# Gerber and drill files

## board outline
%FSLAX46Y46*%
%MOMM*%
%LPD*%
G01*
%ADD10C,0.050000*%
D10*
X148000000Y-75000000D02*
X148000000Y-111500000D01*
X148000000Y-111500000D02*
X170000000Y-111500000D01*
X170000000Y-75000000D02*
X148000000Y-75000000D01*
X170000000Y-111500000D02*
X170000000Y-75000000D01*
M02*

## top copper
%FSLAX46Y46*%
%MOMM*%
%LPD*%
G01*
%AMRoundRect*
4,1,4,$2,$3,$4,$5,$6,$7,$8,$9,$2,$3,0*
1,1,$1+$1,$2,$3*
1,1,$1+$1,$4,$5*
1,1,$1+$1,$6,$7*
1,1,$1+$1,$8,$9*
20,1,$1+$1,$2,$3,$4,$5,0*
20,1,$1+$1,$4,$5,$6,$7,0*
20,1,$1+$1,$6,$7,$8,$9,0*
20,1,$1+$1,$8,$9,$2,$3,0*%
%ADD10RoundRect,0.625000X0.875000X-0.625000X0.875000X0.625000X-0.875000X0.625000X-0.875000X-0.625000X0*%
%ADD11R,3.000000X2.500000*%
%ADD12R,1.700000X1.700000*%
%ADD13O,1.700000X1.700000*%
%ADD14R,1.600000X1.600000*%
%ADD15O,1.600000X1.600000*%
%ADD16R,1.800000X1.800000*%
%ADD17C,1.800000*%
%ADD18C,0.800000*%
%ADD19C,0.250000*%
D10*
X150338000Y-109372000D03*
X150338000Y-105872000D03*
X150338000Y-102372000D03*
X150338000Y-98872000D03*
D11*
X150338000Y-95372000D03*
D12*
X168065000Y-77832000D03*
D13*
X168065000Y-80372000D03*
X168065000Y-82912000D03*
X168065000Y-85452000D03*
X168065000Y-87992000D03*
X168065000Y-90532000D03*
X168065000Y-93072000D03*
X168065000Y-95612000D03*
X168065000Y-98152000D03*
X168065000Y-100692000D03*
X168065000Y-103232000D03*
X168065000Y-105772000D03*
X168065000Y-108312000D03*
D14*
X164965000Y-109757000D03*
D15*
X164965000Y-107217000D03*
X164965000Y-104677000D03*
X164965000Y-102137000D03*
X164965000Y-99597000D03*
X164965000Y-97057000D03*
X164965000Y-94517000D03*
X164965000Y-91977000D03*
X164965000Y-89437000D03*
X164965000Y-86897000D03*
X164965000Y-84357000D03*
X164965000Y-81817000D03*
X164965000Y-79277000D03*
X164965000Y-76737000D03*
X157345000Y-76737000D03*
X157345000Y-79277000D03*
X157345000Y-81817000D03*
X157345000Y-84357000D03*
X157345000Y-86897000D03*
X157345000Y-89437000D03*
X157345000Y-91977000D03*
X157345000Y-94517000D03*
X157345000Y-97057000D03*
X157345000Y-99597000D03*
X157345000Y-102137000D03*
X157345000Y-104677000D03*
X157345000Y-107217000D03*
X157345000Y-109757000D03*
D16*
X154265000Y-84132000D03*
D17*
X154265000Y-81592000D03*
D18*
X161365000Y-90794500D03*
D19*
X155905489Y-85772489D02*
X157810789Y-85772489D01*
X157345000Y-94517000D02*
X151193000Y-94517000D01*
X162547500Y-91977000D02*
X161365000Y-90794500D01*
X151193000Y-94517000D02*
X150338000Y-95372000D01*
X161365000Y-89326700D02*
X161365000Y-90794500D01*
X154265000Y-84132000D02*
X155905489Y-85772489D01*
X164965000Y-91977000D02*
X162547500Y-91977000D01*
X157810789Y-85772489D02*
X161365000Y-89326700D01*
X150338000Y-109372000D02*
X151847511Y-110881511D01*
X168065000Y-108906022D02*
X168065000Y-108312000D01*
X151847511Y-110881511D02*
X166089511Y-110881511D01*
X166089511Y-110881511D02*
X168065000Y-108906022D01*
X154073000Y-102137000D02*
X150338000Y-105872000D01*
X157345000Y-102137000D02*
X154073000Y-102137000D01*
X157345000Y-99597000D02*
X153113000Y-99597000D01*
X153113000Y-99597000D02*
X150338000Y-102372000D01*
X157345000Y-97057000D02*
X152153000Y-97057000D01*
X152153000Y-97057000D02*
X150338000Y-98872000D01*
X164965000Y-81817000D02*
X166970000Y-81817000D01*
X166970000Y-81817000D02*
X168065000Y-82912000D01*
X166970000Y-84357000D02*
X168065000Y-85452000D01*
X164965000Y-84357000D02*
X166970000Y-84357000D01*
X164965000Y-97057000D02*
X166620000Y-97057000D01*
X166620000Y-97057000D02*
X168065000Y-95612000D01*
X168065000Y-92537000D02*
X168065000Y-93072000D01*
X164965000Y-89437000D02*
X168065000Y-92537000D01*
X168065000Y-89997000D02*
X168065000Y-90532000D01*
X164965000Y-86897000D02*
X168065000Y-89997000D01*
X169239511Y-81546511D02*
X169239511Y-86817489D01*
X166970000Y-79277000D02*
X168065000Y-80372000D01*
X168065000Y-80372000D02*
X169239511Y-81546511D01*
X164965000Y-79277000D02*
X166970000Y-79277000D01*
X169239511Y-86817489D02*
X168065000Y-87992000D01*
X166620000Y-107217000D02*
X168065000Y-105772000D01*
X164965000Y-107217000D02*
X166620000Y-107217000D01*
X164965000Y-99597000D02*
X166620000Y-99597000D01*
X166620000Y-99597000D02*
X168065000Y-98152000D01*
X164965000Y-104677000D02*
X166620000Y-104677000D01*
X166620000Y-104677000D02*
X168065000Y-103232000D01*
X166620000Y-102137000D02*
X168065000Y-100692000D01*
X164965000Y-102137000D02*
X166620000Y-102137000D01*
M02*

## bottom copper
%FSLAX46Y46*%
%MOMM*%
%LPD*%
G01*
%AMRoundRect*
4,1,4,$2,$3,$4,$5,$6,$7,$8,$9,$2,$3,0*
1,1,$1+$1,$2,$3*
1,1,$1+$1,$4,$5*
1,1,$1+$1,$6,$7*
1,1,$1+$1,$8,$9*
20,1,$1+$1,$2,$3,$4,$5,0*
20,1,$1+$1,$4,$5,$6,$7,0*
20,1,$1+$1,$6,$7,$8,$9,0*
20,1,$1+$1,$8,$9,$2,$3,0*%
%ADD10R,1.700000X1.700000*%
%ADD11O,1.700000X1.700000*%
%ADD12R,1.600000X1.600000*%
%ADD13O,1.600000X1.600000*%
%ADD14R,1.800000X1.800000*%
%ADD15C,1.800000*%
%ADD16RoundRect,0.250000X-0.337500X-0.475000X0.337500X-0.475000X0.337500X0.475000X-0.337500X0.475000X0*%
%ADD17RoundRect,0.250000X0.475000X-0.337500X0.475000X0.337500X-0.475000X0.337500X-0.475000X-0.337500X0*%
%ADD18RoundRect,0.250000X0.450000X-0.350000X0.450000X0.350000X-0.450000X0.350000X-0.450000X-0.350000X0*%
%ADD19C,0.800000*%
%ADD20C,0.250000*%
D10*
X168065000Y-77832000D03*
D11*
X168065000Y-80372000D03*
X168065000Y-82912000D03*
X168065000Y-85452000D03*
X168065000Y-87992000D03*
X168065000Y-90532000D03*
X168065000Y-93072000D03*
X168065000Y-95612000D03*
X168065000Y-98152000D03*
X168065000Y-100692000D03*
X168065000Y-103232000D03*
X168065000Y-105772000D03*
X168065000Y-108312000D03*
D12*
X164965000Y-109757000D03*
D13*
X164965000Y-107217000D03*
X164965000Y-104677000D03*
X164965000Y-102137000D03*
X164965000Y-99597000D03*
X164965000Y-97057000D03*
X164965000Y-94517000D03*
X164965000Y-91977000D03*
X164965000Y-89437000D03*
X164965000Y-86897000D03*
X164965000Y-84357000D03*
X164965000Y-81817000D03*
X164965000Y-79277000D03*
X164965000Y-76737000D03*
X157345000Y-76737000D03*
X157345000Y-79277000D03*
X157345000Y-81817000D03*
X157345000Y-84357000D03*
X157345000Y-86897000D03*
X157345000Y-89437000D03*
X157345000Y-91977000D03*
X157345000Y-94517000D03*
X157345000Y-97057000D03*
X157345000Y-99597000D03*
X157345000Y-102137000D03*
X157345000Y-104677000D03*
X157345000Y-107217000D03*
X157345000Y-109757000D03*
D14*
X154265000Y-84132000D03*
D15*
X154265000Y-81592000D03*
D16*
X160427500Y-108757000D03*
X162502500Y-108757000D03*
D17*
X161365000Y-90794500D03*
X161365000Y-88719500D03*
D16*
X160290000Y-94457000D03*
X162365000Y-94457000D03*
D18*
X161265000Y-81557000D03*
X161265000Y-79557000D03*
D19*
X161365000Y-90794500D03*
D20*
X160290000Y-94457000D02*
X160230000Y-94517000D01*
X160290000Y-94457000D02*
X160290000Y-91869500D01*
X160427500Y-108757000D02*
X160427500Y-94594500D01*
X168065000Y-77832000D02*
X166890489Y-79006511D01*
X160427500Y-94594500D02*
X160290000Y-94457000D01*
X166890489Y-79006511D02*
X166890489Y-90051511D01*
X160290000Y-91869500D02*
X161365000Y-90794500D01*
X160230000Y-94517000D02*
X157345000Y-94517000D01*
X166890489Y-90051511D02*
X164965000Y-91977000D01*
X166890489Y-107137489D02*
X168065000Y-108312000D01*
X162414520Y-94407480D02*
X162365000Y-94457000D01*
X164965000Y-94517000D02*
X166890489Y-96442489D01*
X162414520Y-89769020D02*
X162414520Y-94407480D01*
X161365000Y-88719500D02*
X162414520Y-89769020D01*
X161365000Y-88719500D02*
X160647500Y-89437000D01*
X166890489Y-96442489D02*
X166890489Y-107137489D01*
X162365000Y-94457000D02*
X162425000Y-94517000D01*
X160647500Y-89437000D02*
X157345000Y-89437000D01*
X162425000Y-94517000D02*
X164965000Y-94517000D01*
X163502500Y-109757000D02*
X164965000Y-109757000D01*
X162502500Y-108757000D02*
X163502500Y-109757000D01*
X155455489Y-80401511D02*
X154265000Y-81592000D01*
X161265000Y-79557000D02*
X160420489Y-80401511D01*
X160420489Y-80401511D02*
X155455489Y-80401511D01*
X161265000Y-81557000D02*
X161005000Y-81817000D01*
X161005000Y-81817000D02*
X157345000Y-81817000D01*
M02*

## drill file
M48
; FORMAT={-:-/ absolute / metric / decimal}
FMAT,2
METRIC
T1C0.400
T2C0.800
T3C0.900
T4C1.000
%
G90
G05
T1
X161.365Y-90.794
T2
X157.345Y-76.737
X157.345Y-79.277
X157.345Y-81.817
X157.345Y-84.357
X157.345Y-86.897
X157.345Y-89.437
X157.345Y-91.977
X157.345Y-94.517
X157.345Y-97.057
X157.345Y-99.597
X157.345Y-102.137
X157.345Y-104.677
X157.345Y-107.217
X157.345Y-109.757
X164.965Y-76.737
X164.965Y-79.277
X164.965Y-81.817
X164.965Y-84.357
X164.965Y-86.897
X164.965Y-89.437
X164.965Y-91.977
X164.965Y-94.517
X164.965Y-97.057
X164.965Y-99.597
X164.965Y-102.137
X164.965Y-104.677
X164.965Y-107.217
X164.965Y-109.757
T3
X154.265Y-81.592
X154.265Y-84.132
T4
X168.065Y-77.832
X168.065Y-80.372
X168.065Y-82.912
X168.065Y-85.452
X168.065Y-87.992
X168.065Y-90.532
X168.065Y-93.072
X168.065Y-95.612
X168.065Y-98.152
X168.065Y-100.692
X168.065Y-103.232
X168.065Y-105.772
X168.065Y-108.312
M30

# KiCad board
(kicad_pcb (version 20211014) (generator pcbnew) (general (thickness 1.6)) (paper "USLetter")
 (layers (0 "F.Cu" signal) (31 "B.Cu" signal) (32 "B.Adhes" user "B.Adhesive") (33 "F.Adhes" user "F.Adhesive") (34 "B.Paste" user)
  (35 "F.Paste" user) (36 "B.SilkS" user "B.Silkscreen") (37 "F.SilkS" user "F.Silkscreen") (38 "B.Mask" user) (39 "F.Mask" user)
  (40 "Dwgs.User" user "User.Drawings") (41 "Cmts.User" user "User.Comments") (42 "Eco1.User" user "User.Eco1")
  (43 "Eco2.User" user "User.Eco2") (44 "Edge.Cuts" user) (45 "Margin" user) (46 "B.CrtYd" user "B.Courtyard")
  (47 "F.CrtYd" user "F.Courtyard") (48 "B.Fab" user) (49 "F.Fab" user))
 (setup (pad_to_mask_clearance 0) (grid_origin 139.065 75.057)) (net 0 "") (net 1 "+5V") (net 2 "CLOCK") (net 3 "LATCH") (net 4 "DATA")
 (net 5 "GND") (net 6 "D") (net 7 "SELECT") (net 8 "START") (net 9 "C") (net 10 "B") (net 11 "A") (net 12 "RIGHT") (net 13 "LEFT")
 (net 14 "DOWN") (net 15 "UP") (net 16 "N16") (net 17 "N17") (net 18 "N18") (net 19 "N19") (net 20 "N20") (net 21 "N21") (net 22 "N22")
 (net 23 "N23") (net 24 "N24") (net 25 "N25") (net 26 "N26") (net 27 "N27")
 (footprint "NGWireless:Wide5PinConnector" (layer "F.Cu") (at 150.465 102.357 90)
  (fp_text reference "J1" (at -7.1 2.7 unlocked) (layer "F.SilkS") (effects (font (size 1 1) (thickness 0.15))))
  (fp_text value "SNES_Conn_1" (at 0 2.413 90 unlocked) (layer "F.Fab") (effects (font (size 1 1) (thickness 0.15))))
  (pad "1" smd roundrect (at -7.015 -0.127 90) (size 2.5 3) (layers "F.Cu" "F.Paste" "F.Mask") (roundrect_rratio 0.25) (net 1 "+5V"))
  (pad "2" smd roundrect (at -3.515 -0.127 90) (size 2.5 3) (layers "F.Cu" "F.Paste" "F.Mask") (roundrect_rratio 0.25) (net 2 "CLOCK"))
  (pad "3" smd roundrect (at -0.015 -0.127 90) (size 2.5 3) (layers "F.Cu" "F.Paste" "F.Mask") (roundrect_rratio 0.25) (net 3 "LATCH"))
  (pad "4" smd roundrect (at 3.485 -0.127 90) (size 2.5 3) (layers "F.Cu" "F.Paste" "F.Mask") (roundrect_rratio 0.25) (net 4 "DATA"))
  (pad "5" smd rect (at 6.985 -0.127 90) (size 2.5 3) (layers "F.Cu" "F.Paste" "F.Mask") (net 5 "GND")))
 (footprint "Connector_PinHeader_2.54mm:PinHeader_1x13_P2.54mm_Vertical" (layer "F.Cu") (at 168.065 77.832)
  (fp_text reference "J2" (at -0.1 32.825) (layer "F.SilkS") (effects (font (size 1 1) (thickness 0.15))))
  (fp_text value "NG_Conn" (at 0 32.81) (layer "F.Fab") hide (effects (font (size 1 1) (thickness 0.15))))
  (pad "1" thru_hole rect locked (at 0 0) (size 1.7 1.7) (drill 1) (layers *.Cu *.Mask) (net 5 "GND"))
  (pad "2" thru_hole oval locked (at 0 2.54) (size 1.7 1.7) (drill 1) (layers *.Cu *.Mask) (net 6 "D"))
  (pad "3" thru_hole oval locked (at 0 5.08) (size 1.7 1.7) (drill 1) (layers *.Cu *.Mask) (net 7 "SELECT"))
  (pad "4" thru_hole oval locked (at 0 7.62) (size 1.7 1.7) (drill 1) (layers *.Cu *.Mask) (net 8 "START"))
  (pad "5" thru_hole oval locked (at 0 10.16) (size 1.7 1.7) (drill 1) (layers *.Cu *.Mask) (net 6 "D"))
  (pad "6" thru_hole oval locked (at 0 12.7) (size 1.7 1.7) (drill 1) (layers *.Cu *.Mask) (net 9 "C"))
  (pad "7" thru_hole oval locked (at 0 15.24) (size 1.7 1.7) (drill 1) (layers *.Cu *.Mask) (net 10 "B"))
  (pad "8" thru_hole oval locked (at 0 17.78) (size 1.7 1.7) (drill 1) (layers *.Cu *.Mask) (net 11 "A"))
  (pad "9" thru_hole oval locked (at 0 20.32) (size 1.7 1.7) (drill 1) (layers *.Cu *.Mask) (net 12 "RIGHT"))
  (pad "10" thru_hole oval locked (at 0 22.86) (size 1.7 1.7) (drill 1) (layers *.Cu *.Mask) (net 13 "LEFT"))
  (pad "11" thru_hole oval locked (at 0 25.4) (size 1.7 1.7) (drill 1) (layers *.Cu *.Mask) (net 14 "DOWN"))
  (pad "12" thru_hole oval locked (at 0 27.94) (size 1.7 1.7) (drill 1) (layers *.Cu *.Mask) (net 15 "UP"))
  (pad "13" thru_hole oval locked (at 0 30.48) (size 1.7 1.7) (drill 1) (layers *.Cu *.Mask) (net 1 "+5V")))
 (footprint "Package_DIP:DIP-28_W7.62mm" (layer "F.Cu") (at 164.965 109.757 180)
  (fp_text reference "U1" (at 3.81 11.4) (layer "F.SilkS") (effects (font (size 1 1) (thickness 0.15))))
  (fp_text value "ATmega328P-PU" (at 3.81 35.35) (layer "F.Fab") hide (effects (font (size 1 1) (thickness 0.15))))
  (pad "1" thru_hole rect locked (at 0 0 180) (size 1.6 1.6) (drill 0.8) (layers *.Cu *.Mask) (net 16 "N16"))
  (pad "2" thru_hole oval locked (at 0 2.54 180) (size 1.6 1.6) (drill 0.8) (layers *.Cu *.Mask) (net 15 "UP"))
  (pad "3" thru_hole oval locked (at 0 5.08 180) (size 1.6 1.6) (drill 0.8) (layers *.Cu *.Mask) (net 14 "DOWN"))
  (pad "4" thru_hole oval locked (at 0 7.62 180) (size 1.6 1.6) (drill 0.8) (layers *.Cu *.Mask) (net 13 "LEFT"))
  (pad "5" thru_hole oval locked (at 0 10.16 180) (size 1.6 1.6) (drill 0.8) (layers *.Cu *.Mask) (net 12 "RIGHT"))
  (pad "6" thru_hole oval locked (at 0 12.7 180) (size 1.6 1.6) (drill 0.8) (layers *.Cu *.Mask) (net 11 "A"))
  (pad "7" thru_hole oval locked (at 0 15.24 180) (size 1.6 1.6) (drill 0.8) (layers *.Cu *.Mask) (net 1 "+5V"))
  (pad "8" thru_hole oval locked (at 0 17.78 180) (size 1.6 1.6) (drill 0.8) (layers *.Cu *.Mask) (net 5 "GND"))
  (pad "9" thru_hole oval locked (at 0 20.32 180) (size 1.6 1.6) (drill 0.8) (layers *.Cu *.Mask) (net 10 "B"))
  (pad "10" thru_hole oval locked (at 0 22.86 180) (size 1.6 1.6) (drill 0.8) (layers *.Cu *.Mask) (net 9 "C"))
  (pad "11" thru_hole oval locked (at 0 25.4 180) (size 1.6 1.6) (drill 0.8) (layers *.Cu *.Mask) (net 8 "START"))
  (pad "12" thru_hole oval locked (at 0 27.94 180) (size 1.6 1.6) (drill 0.8) (layers *.Cu *.Mask) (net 7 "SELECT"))
  (pad "13" thru_hole oval locked (at 0 30.48 180) (size 1.6 1.6) (drill 0.8) (layers *.Cu *.Mask) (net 6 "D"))
  (pad "14" thru_hole oval locked (at 0 33.02 180) (size 1.6 1.6) (drill 0.8) (layers *.Cu *.Mask) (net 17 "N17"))
  (pad "15" thru_hole oval locked (at 7.62 33.02 180) (size 1.6 1.6) (drill 0.8) (layers *.Cu *.Mask) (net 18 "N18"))
  (pad "16" thru_hole oval locked (at 7.62 30.48 180) (size 1.6 1.6) (drill 0.8) (layers *.Cu *.Mask) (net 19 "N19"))
  (pad "17" thru_hole oval locked (at 7.62 27.94 180) (size 1.6 1.6) (drill 0.8) (layers *.Cu *.Mask) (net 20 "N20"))
  (pad "18" thru_hole oval locked (at 7.62 25.4 180) (size 1.6 1.6) (drill 0.8) (layers *.Cu *.Mask) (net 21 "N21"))
  (pad "19" thru_hole oval locked (at 7.62 22.86 180) (size 1.6 1.6) (drill 0.8) (layers *.Cu *.Mask) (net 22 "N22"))
  (pad "20" thru_hole oval locked (at 7.62 20.32 180) (size 1.6 1.6) (drill 0.8) (layers *.Cu *.Mask) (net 1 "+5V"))
  (pad "21" thru_hole oval locked (at 7.62 17.78 180) (size 1.6 1.6) (drill 0.8) (layers *.Cu *.Mask) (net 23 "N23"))
  (pad "22" thru_hole oval locked (at 7.62 15.24 180) (size 1.6 1.6) (drill 0.8) (layers *.Cu *.Mask) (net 5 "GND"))
  (pad "23" thru_hole oval locked (at 7.62 12.7 180) (size 1.6 1.6) (drill 0.8) (layers *.Cu *.Mask) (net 4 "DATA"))
  (pad "24" thru_hole oval locked (at 7.62 10.16 180) (size 1.6 1.6) (drill 0.8) (layers *.Cu *.Mask) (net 3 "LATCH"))
  (pad "25" thru_hole oval locked (at 7.62 7.62 180) (size 1.6 1.6) (drill 0.8) (layers *.Cu *.Mask) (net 2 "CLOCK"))
  (pad "26" thru_hole oval locked (at 7.62 5.08 180) (size 1.6 1.6) (drill 0.8) (layers *.Cu *.Mask) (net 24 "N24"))
  (pad "27" thru_hole oval locked (at 7.62 2.54 180) (size 1.6 1.6) (drill 0.8) (layers *.Cu *.Mask) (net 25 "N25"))
  (pad "28" thru_hole oval locked (at 7.62 0 180) (size 1.6 1.6) (drill 0.8) (layers *.Cu *.Mask) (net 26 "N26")))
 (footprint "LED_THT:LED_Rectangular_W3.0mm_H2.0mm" (layer "F.Cu") (at 154.265 84.132 90)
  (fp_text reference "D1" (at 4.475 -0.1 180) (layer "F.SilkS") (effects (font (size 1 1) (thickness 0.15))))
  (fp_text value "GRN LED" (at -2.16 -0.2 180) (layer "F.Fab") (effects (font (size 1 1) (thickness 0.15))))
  (pad "1" thru_hole rect locked (at 0 0 90) (size 1.8 1.8) (drill 0.9) (layers *.Cu *.Mask) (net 5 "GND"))
  (pad "2" thru_hole circle locked (at 2.54 0 90) (size 1.8 1.8) (drill 0.9) (layers *.Cu *.Mask) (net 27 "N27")))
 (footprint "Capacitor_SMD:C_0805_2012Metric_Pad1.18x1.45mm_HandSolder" (layer "B.Cu") (at 161.465 108.757)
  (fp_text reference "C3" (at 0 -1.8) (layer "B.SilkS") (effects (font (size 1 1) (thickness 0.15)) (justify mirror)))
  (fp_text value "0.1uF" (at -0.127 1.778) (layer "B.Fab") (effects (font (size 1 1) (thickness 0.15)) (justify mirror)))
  (pad "1" smd roundrect locked (at -1.0375 0) (size 1.175 1.45) (layers "B.Cu" "B.Paste" "B.Mask") (roundrect_rratio 0.2127659574)
   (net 5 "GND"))
  (pad "2" smd roundrect locked (at 1.0375 0) (size 1.175 1.45) (layers "B.Cu" "B.Paste" "B.Mask") (roundrect_rratio 0.2127659574)
   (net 16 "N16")))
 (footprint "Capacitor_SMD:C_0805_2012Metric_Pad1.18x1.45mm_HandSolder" (layer "B.Cu") (at 161.365 89.757 90)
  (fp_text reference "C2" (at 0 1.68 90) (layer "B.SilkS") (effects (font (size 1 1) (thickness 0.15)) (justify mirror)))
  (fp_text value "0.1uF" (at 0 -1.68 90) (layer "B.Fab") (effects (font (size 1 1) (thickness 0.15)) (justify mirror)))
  (pad "1" smd roundrect locked (at -1.0375 0 90) (size 1.175 1.45) (layers "B.Cu" "B.Paste" "B.Mask") (roundrect_rratio 0.212766)
   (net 5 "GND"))
  (pad "2" smd roundrect locked (at 1.0375 0 90) (size 1.175 1.45) (layers "B.Cu" "B.Paste" "B.Mask") (roundrect_rratio 0.212766)
   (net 1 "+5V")))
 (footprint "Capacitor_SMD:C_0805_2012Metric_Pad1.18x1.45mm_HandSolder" (layer "B.Cu") (at 161.3275 94.457)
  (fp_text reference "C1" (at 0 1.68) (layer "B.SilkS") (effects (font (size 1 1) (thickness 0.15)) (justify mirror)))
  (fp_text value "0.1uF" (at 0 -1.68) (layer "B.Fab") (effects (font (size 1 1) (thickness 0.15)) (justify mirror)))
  (pad "1" smd roundrect locked (at -1.0375 0) (size 1.175 1.45) (layers "B.Cu" "B.Paste" "B.Mask") (roundrect_rratio 0.212766)
   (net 5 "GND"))
  (pad "2" smd roundrect locked (at 1.0375 0) (size 1.175 1.45) (layers "B.Cu" "B.Paste" "B.Mask") (roundrect_rratio 0.212766) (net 1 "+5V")))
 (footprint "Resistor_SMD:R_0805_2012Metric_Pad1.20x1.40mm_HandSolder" (layer "B.Cu") (at 161.265 80.557 90)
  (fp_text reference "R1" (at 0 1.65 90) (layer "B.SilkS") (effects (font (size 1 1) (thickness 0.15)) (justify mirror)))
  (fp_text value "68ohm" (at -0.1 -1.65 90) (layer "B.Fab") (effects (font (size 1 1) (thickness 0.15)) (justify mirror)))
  (pad "1" smd roundrect locked (at -1 0 90) (size 1.2 1.4) (layers "B.Cu" "B.Paste" "B.Mask") (roundrect_rratio 0.208333) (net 20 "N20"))
  (pad "2" smd roundrect locked (at 1 0 90) (size 1.2 1.4) (layers "B.Cu" "B.Paste" "B.Mask") (roundrect_rratio 0.208333) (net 27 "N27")))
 (gr_line (start 148 75) (end 148 111.5) (layer "Edge.Cuts") (width 0.05))
 (gr_line (start 148 111.5) (end 170 111.5) (layer "Edge.Cuts") (width 0.05))
 (gr_line (start 170 75) (end 148 75) (layer "Edge.Cuts") (width 0.05))
 (gr_line (start 170 111.5) (end 170 75) (layer "Edge.Cuts") (width 0.05))
 (segment (start 155.905489 85.772489) (end 157.810789 85.772489) (width 0.25) (layer "F.Cu") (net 5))
 (segment (start 157.345 94.517) (end 151.193 94.517) (width 0.25) (layer "F.Cu") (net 5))
 (segment (start 162.5475 91.977) (end 161.365 90.7945) (width 0.25) (layer "F.Cu") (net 5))
 (segment (start 151.193 94.517) (end 150.338 95.372) (width 0.25) (layer "F.Cu") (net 5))
 (segment (start 161.365 89.3267) (end 161.365 90.7945) (width 0.25) (layer "F.Cu") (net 5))
 (segment (start 154.265 84.132) (end 155.905489 85.772489) (width 0.25) (layer "F.Cu") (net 5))
 (segment (start 164.965 91.977) (end 162.5475 91.977) (width 0.25) (layer "F.Cu") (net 5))
 (segment (start 157.810789 85.772489) (end 161.365 89.3267) (width 0.25) (layer "F.Cu") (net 5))
 (via (at 161.365 90.7945) (size 0.8) (drill 0.4) (layers "F.Cu" "B.Cu") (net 5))
 (segment (start 160.29 94.457) (end 160.23 94.517) (width 0.25) (layer "B.Cu") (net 5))
 (segment (start 160.29 94.457) (end 160.29 91.8695) (width 0.25) (layer "B.Cu") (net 5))
 (segment (start 160.4275 108.757) (end 160.4275 94.5945) (width 0.25) (layer "B.Cu") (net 5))
 (segment (start 168.065 77.832) (end 166.890489 79.006511) (width 0.25) (layer "B.Cu") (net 5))
 (segment (start 160.4275 94.5945) (end 160.29 94.457) (width 0.25) (layer "B.Cu") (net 5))
 (segment (start 166.890489 79.006511) (end 166.890489 90.051511) (width 0.25) (layer "B.Cu") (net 5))
 (segment (start 160.29 91.8695) (end 161.365 90.7945) (width 0.25) (layer "B.Cu") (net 5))
 (segment (start 160.23 94.517) (end 157.345 94.517) (width 0.25) (layer "B.Cu") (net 5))
 (segment (start 166.890489 90.051511) (end 164.965 91.977) (width 0.25) (layer "B.Cu") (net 5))
 (segment (start 150.338 109.372) (end 151.847511 110.881511) (width 0.25) (layer "F.Cu") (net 1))
 (segment (start 168.065 108.906022) (end 168.065 108.312) (width 0.25) (layer "F.Cu") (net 1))
 (segment (start 151.847511 110.881511) (end 166.089511 110.881511) (width 0.25) (layer "F.Cu") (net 1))
 (segment (start 166.089511 110.881511) (end 168.065 108.906022) (width 0.25) (layer "F.Cu") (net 1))
 (segment (start 166.890489 107.137489) (end 168.065 108.312) (width 0.25) (layer "B.Cu") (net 1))
 (segment (start 162.41452 94.40748) (end 162.365 94.457) (width 0.25) (layer "B.Cu") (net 1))
 (segment (start 164.965 94.517) (end 166.890489 96.442489) (width 0.25) (layer "B.Cu") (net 1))
 (segment (start 162.41452 89.76902) (end 162.41452 94.40748) (width 0.25) (layer "B.Cu") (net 1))
 (segment (start 161.365 88.7195) (end 162.41452 89.76902) (width 0.25) (layer "B.Cu") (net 1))
 (segment (start 161.365 88.7195) (end 160.6475 89.437) (width 0.25) (layer "B.Cu") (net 1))
 (segment (start 166.890489 96.442489) (end 166.890489 107.137489) (width 0.25) (layer "B.Cu") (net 1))
 (segment (start 162.365 94.457) (end 162.425 94.517) (width 0.25) (layer "B.Cu") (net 1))
 (segment (start 160.6475 89.437) (end 157.345 89.437) (width 0.25) (layer "B.Cu") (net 1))
 (segment (start 162.425 94.517) (end 164.965 94.517) (width 0.25) (layer "B.Cu") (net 1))
 (segment (start 154.073 102.137) (end 150.338 105.872) (width 0.25) (layer "F.Cu") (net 2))
 (segment (start 157.345 102.137) (end 154.073 102.137) (width 0.25) (layer "F.Cu") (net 2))
 (segment (start 157.345 99.597) (end 153.113 99.597) (width 0.25) (layer "F.Cu") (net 3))
 (segment (start 153.113 99.597) (end 150.338 102.372) (width 0.25) (layer "F.Cu") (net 3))
 (segment (start 157.345 97.057) (end 152.153 97.057) (width 0.25) (layer "F.Cu") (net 4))
 (segment (start 152.153 97.057) (end 150.338 98.872) (width 0.25) (layer "F.Cu") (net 4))
 (segment (start 164.965 81.817) (end 166.97 81.817) (width 0.25) (layer "F.Cu") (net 7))
 (segment (start 166.97 81.817) (end 168.065 82.912) (width 0.25) (layer "F.Cu") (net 7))
 (segment (start 166.97 84.357) (end 168.065 85.452) (width 0.25) (layer "F.Cu") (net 8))
 (segment (start 164.965 84.357) (end 166.97 84.357) (width 0.25) (layer "F.Cu") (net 8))
 (segment (start 164.965 97.057) (end 166.62 97.057) (width 0.25) (layer "F.Cu") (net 11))
 (segment (start 166.62 97.057) (end 168.065 95.612) (width 0.25) (layer "F.Cu") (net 11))
 (segment (start 168.065 92.537) (end 168.065 93.072) (width 0.25) (layer "F.Cu") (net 10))
 (segment (start 164.965 89.437) (end 168.065 92.537) (width 0.25) (layer "F.Cu") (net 10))
 (segment (start 168.065 89.997) (end 168.065 90.532) (width 0.25) (layer "F.Cu") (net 9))
 (segment (start 164.965 86.897) (end 168.065 89.997) (width 0.25) (layer "F.Cu") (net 9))
 (segment (start 169.239511 81.546511) (end 169.239511 86.817489) (width 0.25) (layer "F.Cu") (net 6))
 (segment (start 166.97 79.277) (end 168.065 80.372) (width 0.25) (layer "F.Cu") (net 6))
 (segment (start 168.065 80.372) (end 169.239511 81.546511) (width 0.25) (layer "F.Cu") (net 6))
 (segment (start 164.965 79.277) (end 166.97 79.277) (width 0.25) (layer "F.Cu") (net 6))
 (segment (start 169.239511 86.817489) (end 168.065 87.992) (width 0.25) (layer "F.Cu") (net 6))
 (segment (start 166.62 107.217) (end 168.065 105.772) (width 0.25) (layer "F.Cu") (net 15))
 (segment (start 164.965 107.217) (end 166.62 107.217) (width 0.25) (layer "F.Cu") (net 15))
 (segment (start 164.965 99.597) (end 166.62 99.597) (width 0.25) (layer "F.Cu") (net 12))
 (segment (start 166.62 99.597) (end 168.065 98.152) (width 0.25) (layer "F.Cu") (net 12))
 (segment (start 164.965 104.677) (end 166.62 104.677) (width 0.25) (layer "F.Cu") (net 14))
 (segment (start 166.62 104.677) (end 168.065 103.232) (width 0.25) (layer "F.Cu") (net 14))
 (segment (start 166.62 102.137) (end 168.065 100.692) (width 0.25) (layer "F.Cu") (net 13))
 (segment (start 164.965 102.137) (end 166.62 102.137) (width 0.25) (layer "F.Cu") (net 13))
 (segment (start 163.5025 109.757) (end 164.965 109.757) (width 0.25) (layer "B.Cu") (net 16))
 (segment (start 162.5025 108.757) (end 163.5025 109.757) (width 0.25) (layer "B.Cu") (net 16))
 (segment (start 155.455489 80.401511) (end 154.265 81.592) (width 0.25) (layer "B.Cu") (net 27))
 (segment (start 161.265 79.557) (end 160.420489 80.401511) (width 0.25) (layer "B.Cu") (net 27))
 (segment (start 160.420489 80.401511) (end 155.455489 80.401511) (width 0.25) (layer "B.Cu") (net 27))
 (segment (start 161.265 81.557) (end 161.005 81.817) (width 0.25) (layer "B.Cu") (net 20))
 (segment (start 161.005 81.817) (end 157.345 81.817) (width 0.25) (layer "B.Cu") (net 20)))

